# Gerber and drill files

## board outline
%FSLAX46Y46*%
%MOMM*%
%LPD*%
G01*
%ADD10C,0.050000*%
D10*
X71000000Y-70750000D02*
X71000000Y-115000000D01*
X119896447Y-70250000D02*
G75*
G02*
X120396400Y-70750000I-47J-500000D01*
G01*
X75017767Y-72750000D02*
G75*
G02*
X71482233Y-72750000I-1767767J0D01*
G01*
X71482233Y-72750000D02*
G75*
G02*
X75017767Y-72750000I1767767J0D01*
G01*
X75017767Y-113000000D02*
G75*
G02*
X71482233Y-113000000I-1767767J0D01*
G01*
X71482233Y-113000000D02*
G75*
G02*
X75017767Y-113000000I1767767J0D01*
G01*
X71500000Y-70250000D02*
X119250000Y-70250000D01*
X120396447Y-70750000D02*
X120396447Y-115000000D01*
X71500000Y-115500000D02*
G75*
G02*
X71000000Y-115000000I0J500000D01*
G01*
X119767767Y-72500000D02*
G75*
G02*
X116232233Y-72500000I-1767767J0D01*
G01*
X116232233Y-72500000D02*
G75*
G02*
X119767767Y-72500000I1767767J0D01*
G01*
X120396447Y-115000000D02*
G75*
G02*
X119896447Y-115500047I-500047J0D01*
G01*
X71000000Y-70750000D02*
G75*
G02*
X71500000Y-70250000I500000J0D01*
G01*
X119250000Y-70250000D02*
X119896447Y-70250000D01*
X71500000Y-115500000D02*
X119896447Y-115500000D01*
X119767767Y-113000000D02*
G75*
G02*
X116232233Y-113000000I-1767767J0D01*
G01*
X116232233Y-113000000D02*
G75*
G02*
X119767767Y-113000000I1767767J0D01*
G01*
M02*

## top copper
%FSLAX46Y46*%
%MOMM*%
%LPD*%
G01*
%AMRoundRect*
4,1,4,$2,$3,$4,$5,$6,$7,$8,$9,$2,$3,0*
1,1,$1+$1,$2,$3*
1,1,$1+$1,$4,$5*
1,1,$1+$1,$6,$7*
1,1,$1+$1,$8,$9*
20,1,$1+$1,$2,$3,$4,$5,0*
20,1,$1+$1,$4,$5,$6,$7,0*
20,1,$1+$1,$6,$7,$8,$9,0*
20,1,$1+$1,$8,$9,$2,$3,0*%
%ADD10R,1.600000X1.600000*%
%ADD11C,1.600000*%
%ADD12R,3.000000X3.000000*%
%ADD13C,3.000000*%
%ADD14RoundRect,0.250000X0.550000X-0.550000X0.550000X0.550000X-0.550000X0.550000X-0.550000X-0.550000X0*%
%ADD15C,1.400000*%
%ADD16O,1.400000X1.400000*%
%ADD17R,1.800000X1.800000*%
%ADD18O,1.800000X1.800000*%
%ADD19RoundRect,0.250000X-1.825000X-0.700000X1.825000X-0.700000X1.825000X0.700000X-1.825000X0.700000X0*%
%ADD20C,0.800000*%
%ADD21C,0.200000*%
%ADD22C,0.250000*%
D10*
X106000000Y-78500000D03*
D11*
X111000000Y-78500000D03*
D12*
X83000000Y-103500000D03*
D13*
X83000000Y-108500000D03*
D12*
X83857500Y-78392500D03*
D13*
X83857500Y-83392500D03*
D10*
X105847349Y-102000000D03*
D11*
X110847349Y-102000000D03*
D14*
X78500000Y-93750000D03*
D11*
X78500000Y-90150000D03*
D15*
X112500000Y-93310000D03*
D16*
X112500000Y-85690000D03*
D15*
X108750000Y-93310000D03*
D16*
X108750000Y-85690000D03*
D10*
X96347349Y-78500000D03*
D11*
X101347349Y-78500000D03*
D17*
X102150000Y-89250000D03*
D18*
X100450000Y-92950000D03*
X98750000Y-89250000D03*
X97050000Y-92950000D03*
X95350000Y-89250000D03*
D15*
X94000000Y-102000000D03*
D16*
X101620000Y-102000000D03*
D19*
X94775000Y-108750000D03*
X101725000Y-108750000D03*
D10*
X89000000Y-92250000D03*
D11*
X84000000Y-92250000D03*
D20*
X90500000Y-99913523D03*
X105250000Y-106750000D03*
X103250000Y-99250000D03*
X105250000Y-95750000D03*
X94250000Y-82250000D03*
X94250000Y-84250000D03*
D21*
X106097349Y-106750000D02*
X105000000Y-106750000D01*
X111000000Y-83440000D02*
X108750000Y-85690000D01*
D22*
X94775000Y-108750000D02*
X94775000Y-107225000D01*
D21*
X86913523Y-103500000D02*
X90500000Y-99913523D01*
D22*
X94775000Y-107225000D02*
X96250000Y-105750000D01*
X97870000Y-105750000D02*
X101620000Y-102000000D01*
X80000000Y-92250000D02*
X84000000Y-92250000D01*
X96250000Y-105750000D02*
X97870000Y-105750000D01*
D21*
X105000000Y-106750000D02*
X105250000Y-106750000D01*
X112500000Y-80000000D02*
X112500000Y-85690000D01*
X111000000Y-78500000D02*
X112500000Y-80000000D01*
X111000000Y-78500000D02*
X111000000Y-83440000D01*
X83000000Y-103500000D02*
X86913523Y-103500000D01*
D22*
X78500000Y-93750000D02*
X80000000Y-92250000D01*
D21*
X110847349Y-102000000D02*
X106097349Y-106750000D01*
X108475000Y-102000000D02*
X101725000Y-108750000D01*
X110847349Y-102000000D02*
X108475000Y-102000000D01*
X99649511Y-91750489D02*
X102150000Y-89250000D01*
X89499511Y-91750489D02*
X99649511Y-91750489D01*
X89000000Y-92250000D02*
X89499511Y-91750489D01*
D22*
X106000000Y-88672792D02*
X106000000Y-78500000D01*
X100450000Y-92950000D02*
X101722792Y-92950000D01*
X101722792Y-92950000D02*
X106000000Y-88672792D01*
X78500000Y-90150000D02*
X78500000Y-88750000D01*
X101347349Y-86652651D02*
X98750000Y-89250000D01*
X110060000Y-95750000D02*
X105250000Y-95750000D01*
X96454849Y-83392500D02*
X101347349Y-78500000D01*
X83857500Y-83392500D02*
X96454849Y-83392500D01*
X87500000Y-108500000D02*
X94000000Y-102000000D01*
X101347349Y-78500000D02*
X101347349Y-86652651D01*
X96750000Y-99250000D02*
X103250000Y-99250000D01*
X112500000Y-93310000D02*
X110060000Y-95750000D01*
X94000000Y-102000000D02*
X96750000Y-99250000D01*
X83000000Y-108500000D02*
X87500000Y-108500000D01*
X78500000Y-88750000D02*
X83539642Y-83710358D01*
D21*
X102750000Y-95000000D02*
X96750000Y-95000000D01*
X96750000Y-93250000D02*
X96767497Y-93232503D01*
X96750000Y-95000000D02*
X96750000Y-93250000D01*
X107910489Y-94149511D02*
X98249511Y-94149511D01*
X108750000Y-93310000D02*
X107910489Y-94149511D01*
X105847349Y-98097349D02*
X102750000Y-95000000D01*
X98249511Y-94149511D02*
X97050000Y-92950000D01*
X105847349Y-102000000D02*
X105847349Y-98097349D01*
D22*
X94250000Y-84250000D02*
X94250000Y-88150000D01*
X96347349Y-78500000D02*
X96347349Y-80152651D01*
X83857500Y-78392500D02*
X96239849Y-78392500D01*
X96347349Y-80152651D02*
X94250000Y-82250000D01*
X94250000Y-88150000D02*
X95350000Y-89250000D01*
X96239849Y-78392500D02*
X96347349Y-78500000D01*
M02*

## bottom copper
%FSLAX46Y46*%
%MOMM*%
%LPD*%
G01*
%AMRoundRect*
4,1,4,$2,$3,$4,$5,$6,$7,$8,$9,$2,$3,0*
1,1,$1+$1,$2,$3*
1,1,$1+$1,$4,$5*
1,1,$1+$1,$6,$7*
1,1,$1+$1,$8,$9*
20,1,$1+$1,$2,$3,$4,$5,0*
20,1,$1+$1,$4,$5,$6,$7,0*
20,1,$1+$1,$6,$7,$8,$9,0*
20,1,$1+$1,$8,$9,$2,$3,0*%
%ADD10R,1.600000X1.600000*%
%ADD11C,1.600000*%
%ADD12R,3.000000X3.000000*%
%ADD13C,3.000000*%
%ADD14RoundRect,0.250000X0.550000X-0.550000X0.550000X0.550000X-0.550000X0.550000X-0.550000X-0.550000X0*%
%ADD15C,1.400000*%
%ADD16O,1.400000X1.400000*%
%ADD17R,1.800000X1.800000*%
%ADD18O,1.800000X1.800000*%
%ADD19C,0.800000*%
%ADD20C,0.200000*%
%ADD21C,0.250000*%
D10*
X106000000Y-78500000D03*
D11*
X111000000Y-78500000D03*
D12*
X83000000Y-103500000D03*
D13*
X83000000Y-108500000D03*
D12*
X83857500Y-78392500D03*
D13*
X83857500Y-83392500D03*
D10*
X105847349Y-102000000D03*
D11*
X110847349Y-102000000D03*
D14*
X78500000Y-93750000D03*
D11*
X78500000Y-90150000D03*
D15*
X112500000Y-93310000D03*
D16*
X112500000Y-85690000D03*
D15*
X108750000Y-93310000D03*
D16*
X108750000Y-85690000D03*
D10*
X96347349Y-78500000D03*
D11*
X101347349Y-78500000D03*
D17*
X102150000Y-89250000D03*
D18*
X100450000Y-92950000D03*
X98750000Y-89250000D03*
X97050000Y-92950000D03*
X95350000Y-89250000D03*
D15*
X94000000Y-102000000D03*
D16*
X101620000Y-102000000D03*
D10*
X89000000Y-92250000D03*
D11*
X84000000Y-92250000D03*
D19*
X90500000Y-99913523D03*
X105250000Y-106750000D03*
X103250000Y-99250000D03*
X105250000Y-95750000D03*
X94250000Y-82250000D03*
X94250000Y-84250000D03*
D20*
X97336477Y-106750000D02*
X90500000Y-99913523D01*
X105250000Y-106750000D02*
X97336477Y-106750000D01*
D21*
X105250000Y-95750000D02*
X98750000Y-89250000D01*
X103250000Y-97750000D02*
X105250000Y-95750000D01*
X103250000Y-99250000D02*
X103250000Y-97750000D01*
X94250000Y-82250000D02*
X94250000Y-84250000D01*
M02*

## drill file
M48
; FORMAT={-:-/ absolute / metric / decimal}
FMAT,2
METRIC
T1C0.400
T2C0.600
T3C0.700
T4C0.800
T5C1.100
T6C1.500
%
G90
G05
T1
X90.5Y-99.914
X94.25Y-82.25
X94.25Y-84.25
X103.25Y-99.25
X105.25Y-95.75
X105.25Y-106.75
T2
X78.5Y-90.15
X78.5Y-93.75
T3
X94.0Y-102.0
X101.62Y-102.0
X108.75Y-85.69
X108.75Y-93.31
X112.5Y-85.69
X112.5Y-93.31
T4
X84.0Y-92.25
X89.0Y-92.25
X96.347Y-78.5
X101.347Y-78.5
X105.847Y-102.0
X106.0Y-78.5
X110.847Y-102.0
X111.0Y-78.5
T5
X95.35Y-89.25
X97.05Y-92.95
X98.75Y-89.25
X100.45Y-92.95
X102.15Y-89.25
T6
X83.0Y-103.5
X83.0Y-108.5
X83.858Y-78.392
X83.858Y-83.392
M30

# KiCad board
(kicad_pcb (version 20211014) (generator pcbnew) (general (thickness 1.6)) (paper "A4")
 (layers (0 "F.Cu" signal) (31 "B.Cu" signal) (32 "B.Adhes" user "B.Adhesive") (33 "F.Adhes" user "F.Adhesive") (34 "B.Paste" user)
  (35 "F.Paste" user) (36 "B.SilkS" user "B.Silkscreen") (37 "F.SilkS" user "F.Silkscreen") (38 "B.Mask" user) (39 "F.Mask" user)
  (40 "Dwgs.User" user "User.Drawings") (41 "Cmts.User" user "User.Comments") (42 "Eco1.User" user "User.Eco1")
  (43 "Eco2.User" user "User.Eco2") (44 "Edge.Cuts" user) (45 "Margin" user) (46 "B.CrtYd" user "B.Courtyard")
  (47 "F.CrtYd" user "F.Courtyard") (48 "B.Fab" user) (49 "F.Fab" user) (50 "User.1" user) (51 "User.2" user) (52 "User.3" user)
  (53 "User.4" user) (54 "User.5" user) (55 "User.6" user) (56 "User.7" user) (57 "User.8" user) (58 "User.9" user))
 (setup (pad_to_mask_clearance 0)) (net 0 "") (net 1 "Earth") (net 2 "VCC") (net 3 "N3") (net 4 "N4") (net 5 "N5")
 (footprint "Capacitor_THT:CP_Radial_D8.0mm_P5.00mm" (layer "F.Cu") (at 106 78.5)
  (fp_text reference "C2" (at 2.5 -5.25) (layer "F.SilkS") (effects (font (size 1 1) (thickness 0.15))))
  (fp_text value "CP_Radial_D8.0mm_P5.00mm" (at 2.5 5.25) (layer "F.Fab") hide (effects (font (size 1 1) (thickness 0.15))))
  (pad "1" thru_hole rect (at 0 0) (size 1.6 1.6) (drill 0.8) (layers *.Cu *.Mask))
  (pad "2" thru_hole circle (at 5 0) (size 1.6 1.6) (drill 0.8) (layers *.Cu *.Mask)))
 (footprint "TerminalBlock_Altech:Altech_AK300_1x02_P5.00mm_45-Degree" (layer "F.Cu") (at 83 103.5 -90)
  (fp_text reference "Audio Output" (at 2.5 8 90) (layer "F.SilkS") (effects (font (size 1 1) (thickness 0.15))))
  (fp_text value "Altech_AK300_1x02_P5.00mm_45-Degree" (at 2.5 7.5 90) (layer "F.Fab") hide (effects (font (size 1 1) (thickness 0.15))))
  (pad "1" thru_hole rect (at 0 0 270) (size 3 3) (drill 1.5) (layers *.Cu *.Mask))
  (pad "2" thru_hole circle (at 5 0 270) (size 3 3) (drill 1.5) (layers *.Cu *.Mask) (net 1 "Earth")))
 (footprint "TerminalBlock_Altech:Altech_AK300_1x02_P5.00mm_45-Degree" (layer "F.Cu") (at 83.8575 78.3925 -90)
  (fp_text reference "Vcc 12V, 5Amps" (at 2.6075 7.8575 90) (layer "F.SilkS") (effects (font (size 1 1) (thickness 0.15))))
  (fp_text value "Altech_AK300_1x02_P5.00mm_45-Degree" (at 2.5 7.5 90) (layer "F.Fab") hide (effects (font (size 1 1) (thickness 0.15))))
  (pad "1" thru_hole rect (at 0 0 270) (size 3 3) (drill 1.5) (layers *.Cu *.Mask) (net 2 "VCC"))
  (pad "2" thru_hole circle (at 5 0 270) (size 3 3) (drill 1.5) (layers *.Cu *.Mask) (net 1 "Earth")))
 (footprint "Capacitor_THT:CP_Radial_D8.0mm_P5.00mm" (layer "F.Cu") (at 105.847349 102)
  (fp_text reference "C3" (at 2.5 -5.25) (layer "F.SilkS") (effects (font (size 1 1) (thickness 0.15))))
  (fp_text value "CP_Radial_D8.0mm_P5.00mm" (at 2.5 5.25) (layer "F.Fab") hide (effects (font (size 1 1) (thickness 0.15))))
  (pad "1" thru_hole rect (at 0 0) (size 1.6 1.6) (drill 0.8) (layers *.Cu *.Mask) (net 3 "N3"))
  (pad "2" thru_hole circle (at 5 0) (size 1.6 1.6) (drill 0.8) (layers *.Cu *.Mask)))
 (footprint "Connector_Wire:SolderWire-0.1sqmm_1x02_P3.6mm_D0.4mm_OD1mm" (layer "F.Cu") (at 78.5 93.75 90)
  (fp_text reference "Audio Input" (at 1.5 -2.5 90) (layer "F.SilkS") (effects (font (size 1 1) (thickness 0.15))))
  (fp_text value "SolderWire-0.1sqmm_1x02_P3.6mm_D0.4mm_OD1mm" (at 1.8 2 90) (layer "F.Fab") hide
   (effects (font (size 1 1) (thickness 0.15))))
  (pad "1" thru_hole roundrect (at 0 0 90) (size 1.6 1.6) (drill 0.6) (layers *.Cu *.Mask) (roundrect_rratio 0.15625))
  (pad "2" thru_hole circle (at 3.6 0 90) (size 1.6 1.6) (drill 0.6) (layers *.Cu *.Mask) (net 1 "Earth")))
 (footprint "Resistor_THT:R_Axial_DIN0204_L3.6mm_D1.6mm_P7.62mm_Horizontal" (layer "F.Cu") (at 112.5 93.31 90)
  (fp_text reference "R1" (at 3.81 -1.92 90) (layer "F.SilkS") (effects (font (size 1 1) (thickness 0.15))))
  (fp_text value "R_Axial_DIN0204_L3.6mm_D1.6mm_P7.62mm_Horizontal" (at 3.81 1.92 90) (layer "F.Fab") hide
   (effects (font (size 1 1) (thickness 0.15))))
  (pad "1" thru_hole circle (at 0 0 90) (size 1.4 1.4) (drill 0.7) (layers *.Cu *.Mask) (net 1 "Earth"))
  (pad "2" thru_hole oval (at 7.62 0 90) (size 1.4 1.4) (drill 0.7) (layers *.Cu *.Mask)))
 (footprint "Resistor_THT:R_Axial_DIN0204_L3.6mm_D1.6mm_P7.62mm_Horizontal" (layer "F.Cu") (at 108.75 93.31 90)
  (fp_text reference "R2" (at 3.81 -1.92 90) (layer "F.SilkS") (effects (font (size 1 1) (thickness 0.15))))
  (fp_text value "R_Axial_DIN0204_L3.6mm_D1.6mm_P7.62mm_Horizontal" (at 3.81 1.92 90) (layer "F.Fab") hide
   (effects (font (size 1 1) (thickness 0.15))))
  (pad "1" thru_hole circle (at 0 0 90) (size 1.4 1.4) (drill 0.7) (layers *.Cu *.Mask))
  (pad "2" thru_hole oval (at 7.62 0 90) (size 1.4 1.4) (drill 0.7) (layers *.Cu *.Mask)))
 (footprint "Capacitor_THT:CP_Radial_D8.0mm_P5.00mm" (layer "F.Cu") (at 96.347349 78.5)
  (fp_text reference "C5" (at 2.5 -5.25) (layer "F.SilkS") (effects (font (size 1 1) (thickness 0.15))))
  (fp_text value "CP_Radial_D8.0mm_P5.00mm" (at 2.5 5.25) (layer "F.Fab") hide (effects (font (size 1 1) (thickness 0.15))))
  (pad "1" thru_hole rect (at 0 0) (size 1.6 1.6) (drill 0.8) (layers *.Cu *.Mask))
  (pad "2" thru_hole circle (at 5 0) (size 1.6 1.6) (drill 0.8) (layers *.Cu *.Mask) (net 1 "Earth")))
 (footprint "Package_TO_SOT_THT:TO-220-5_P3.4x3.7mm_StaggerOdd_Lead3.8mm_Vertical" (layer "F.Cu") (at 102.15 89.25 180)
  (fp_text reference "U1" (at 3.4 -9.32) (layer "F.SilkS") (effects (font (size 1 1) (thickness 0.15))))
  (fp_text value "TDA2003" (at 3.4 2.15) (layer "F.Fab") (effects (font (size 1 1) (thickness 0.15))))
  (pad "1" thru_hole rect (at 0 0 180) (size 1.8 1.8) (drill 1.1) (layers *.Cu *.Mask) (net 3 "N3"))
  (pad "2" thru_hole oval (at 1.7 -3.7 180) (size 1.8 1.8) (drill 1.1) (layers *.Cu *.Mask) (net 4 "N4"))
  (pad "3" thru_hole oval (at 3.4 0 180) (size 1.8 1.8) (drill 1.1) (layers *.Cu *.Mask) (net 1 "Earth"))
  (pad "4" thru_hole oval (at 5.1 -3.7 180) (size 1.8 1.8) (drill 1.1) (layers *.Cu *.Mask) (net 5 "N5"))
  (pad "5" thru_hole oval (at 6.8 0 180) (size 1.8 1.8) (drill 1.1) (layers *.Cu *.Mask) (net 2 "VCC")))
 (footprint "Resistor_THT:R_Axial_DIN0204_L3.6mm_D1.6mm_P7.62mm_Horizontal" (layer "F.Cu") (at 94 102)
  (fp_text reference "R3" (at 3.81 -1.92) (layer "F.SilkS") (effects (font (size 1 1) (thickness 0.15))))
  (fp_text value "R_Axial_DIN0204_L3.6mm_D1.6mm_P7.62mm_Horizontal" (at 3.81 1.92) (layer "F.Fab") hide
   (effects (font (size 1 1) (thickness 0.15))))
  (pad "1" thru_hole circle (at 0 0) (size 1.4 1.4) (drill 0.7) (layers *.Cu *.Mask) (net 1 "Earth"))
  (pad "2" thru_hole oval (at 7.62 0) (size 1.4 1.4) (drill 0.7) (layers *.Cu *.Mask)))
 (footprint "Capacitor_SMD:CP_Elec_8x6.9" (layer "F.Cu") (at 98.25 108.75)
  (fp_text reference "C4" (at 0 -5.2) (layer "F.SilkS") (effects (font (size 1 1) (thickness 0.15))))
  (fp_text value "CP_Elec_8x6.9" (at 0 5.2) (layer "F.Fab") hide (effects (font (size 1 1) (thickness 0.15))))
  (pad "1" smd roundrect (at -3.475 0) (size 4.15 1.9) (layers "F.Cu" "F.Paste" "F.Mask") (roundrect_rratio 0.131579))
  (pad "2" smd roundrect (at 3.475 0) (size 4.15 1.9) (layers "F.Cu" "F.Paste" "F.Mask") (roundrect_rratio 0.131579)))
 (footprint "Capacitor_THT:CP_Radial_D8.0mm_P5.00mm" (layer "F.Cu") (at 89 92.25 180)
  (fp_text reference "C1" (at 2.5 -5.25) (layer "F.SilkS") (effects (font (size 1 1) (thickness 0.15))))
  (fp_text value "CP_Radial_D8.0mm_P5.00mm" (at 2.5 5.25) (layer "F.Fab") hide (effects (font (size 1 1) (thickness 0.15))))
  (pad "1" thru_hole rect (at 0 0 180) (size 1.6 1.6) (drill 0.8) (layers *.Cu *.Mask))
  (pad "2" thru_hole circle (at 5 0 180) (size 1.6 1.6) (drill 0.8) (layers *.Cu *.Mask)))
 (gr_line (start 71 70.75) (end 71 115) (layer "Edge.Cuts") (width 0.05))
 (gr_arc (start 119.896447 70.25) (mid 120.25 70.396447) (end 120.396447 70.75) (layer "Edge.Cuts") (width 0.05))
 (gr_circle (center 73.25 72.75) (end 74.5 74) (layer "Edge.Cuts") (width 0.05) (fill none))
 (gr_circle (center 73.25 113) (end 74.5 114.25) (layer "Edge.Cuts") (width 0.05) (fill none))
 (gr_line (start 71.5 70.25) (end 119.25 70.25) (layer "Edge.Cuts") (width 0.05))
 (gr_line (start 120.396447 70.75) (end 120.396447 115) (layer "Edge.Cuts") (width 0.05))
 (gr_arc (start 71.5 115.5) (mid 71.146447 115.353553) (end 71 115) (layer "Edge.Cuts") (width 0.05))
 (gr_circle (center 118 72.5) (end 119.25 73.75) (layer "Edge.Cuts") (width 0.05) (fill none))
 (gr_arc (start 120.396447 115) (mid 120.25 115.353553) (end 119.896447 115.5) (layer "Edge.Cuts") (width 0.05))
 (gr_arc (start 71 70.75) (mid 71.146447 70.396447) (end 71.5 70.25) (layer "Edge.Cuts") (width 0.05))
 (gr_line (start 119.25 70.25) (end 119.896447 70.25) (layer "Edge.Cuts") (width 0.05))
 (gr_line (start 71.5 115.5) (end 119.896447 115.5) (layer "Edge.Cuts") (width 0.05))
 (gr_circle (center 118 113) (end 119.25 114.25) (layer "Edge.Cuts") (width 0.05) (fill none))
 (segment (start 106.097349 106.75) (end 105 106.75) (width 0.2) (layer "F.Cu") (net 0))
 (segment (start 111 83.44) (end 108.75 85.69) (width 0.2) (layer "F.Cu") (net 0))
 (segment (start 94.775 108.75) (end 94.775 107.225) (width 0.25) (layer "F.Cu") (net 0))
 (segment (start 86.913523 103.5) (end 90.5 99.913523) (width 0.2) (layer "F.Cu") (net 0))
 (segment (start 94.775 107.225) (end 96.25 105.75) (width 0.25) (layer "F.Cu") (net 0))
 (segment (start 97.87 105.75) (end 101.62 102) (width 0.25) (layer "F.Cu") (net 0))
 (segment (start 80 92.25) (end 84 92.25) (width 0.25) (layer "F.Cu") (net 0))
 (segment (start 96.25 105.75) (end 97.87 105.75) (width 0.25) (layer "F.Cu") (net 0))
 (segment (start 105 106.75) (end 105.25 106.75) (width 0.2) (layer "F.Cu") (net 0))
 (segment (start 112.5 80) (end 112.5 85.69) (width 0.2) (layer "F.Cu") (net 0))
 (segment (start 111 78.5) (end 112.5 80) (width 0.2) (layer "F.Cu") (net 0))
 (segment (start 111 78.5) (end 111 83.44) (width 0.2) (layer "F.Cu") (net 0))
 (segment (start 83 103.5) (end 86.913523 103.5) (width 0.2) (layer "F.Cu") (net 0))
 (segment (start 78.5 93.75) (end 80 92.25) (width 0.25) (layer "F.Cu") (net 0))
 (segment (start 110.847349 102) (end 106.097349 106.75) (width 0.2) (layer "F.Cu") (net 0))
 (segment (start 108.475 102) (end 101.725 108.75) (width 0.2) (layer "F.Cu") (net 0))
 (segment (start 110.847349 102) (end 108.475 102) (width 0.2) (layer "F.Cu") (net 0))
 (via (at 90.5 99.913523) (size 0.8) (drill 0.4) (layers "F.Cu" "B.Cu") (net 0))
 (via (at 105.25 106.75) (size 0.8) (drill 0.4) (layers "F.Cu" "B.Cu") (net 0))
 (segment (start 97.336477 106.75) (end 90.5 99.913523) (width 0.2) (layer "B.Cu") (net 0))
 (segment (start 105.25 106.75) (end 97.336477 106.75) (width 0.2) (layer "B.Cu") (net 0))
 (segment (start 99.649511 91.750489) (end 102.15 89.25) (width 0.2) (layer "F.Cu") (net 3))
 (segment (start 89.499511 91.750489) (end 99.649511 91.750489) (width 0.2) (layer "F.Cu") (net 3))
 (segment (start 89 92.25) (end 89.499511 91.750489) (width 0.2) (layer "F.Cu") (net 3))
 (segment (start 106 88.672792) (end 106 78.5) (width 0.25) (layer "F.Cu") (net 4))
 (segment (start 100.45 92.95) (end 101.722792 92.95) (width 0.25) (layer "F.Cu") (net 4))
 (segment (start 101.722792 92.95) (end 106 88.672792) (width 0.25) (layer "F.Cu") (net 4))
 (segment (start 78.5 90.15) (end 78.5 88.75) (width 0.25) (layer "F.Cu") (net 1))
 (segment (start 101.347349 86.652651) (end 98.75 89.25) (width 0.25) (layer "F.Cu") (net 1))
 (segment (start 110.06 95.75) (end 105.25 95.75) (width 0.25) (layer "F.Cu") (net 1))
 (segment (start 96.454849 83.3925) (end 101.347349 78.5) (width 0.25) (layer "F.Cu") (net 1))
 (segment (start 83.8575 83.3925) (end 96.454849 83.3925) (width 0.25) (layer "F.Cu") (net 1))
 (segment (start 87.5 108.5) (end 94 102) (width 0.25) (layer "F.Cu") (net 1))
 (segment (start 101.347349 78.5) (end 101.347349 86.652651) (width 0.25) (layer "F.Cu") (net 1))
 (segment (start 96.75 99.25) (end 103.25 99.25) (width 0.25) (layer "F.Cu") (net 1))
 (segment (start 112.5 93.31) (end 110.06 95.75) (width 0.25) (layer "F.Cu") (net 1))
 (segment (start 94 102) (end 96.75 99.25) (width 0.25) (layer "F.Cu") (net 1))
 (segment (start 83 108.5) (end 87.5 108.5) (width 0.25) (layer "F.Cu") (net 1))
 (segment (start 78.5 88.75) (end 83.539642 83.710358) (width 0.25) (layer "F.Cu") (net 1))
 (via (at 103.25 99.25) (size 0.8) (drill 0.4) (layers "F.Cu" "B.Cu") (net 1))
 (via (at 105.25 95.75) (size 0.8) (drill 0.4) (layers "F.Cu" "B.Cu") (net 1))
 (segment (start 105.25 95.75) (end 98.75 89.25) (width 0.25) (layer "B.Cu") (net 1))
 (segment (start 103.25 97.75) (end 105.25 95.75) (width 0.25) (layer "B.Cu") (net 1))
 (segment (start 103.25 99.25) (end 103.25 97.75) (width 0.25) (layer "B.Cu") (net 1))
 (segment (start 102.75 95) (end 96.75 95) (width 0.2) (layer "F.Cu") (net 5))
 (segment (start 96.75 93.25) (end 96.767497 93.232503) (width 0.2) (layer "F.Cu") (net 5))
 (segment (start 96.75 95) (end 96.75 93.25) (width 0.2) (layer "F.Cu") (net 5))
 (segment (start 107.910489 94.149511) (end 98.249511 94.149511) (width 0.2) (layer "F.Cu") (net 5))
 (segment (start 108.75 93.31) (end 107.910489 94.149511) (width 0.2) (layer "F.Cu") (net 5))
 (segment (start 105.847349 98.097349) (end 102.75 95) (width 0.2) (layer "F.Cu") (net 5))
 (segment (start 98.249511 94.149511) (end 97.05 92.95) (width 0.2) (layer "F.Cu") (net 5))
 (segment (start 105.847349 102) (end 105.847349 98.097349) (width 0.2) (layer "F.Cu") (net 5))
 (segment (start 94.25 84.25) (end 94.25 88.15) (width 0.25) (layer "F.Cu") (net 2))
 (segment (start 96.347349 78.5) (end 96.347349 80.152651) (width 0.25) (layer "F.Cu") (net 2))
 (segment (start 83.8575 78.3925) (end 96.239849 78.3925) (width 0.25) (layer "F.Cu") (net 2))
 (segment (start 96.347349 80.152651) (end 94.25 82.25) (width 0.25) (layer "F.Cu") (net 2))
 (segment (start 94.25 88.15) (end 95.35 89.25) (width 0.25) (layer "F.Cu") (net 2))
 (segment (start 96.239849 78.3925) (end 96.347349 78.5) (width 0.25) (layer "F.Cu") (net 2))
 (via (at 94.25 82.25) (size 0.8) (drill 0.4) (layers "F.Cu" "B.Cu") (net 2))
 (via (at 94.25 84.25) (size 0.8) (drill 0.4) (layers "F.Cu" "B.Cu") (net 2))
 (segment (start 94.25 82.25) (end 94.25 84.25) (width 0.25) (layer "B.Cu") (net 2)))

